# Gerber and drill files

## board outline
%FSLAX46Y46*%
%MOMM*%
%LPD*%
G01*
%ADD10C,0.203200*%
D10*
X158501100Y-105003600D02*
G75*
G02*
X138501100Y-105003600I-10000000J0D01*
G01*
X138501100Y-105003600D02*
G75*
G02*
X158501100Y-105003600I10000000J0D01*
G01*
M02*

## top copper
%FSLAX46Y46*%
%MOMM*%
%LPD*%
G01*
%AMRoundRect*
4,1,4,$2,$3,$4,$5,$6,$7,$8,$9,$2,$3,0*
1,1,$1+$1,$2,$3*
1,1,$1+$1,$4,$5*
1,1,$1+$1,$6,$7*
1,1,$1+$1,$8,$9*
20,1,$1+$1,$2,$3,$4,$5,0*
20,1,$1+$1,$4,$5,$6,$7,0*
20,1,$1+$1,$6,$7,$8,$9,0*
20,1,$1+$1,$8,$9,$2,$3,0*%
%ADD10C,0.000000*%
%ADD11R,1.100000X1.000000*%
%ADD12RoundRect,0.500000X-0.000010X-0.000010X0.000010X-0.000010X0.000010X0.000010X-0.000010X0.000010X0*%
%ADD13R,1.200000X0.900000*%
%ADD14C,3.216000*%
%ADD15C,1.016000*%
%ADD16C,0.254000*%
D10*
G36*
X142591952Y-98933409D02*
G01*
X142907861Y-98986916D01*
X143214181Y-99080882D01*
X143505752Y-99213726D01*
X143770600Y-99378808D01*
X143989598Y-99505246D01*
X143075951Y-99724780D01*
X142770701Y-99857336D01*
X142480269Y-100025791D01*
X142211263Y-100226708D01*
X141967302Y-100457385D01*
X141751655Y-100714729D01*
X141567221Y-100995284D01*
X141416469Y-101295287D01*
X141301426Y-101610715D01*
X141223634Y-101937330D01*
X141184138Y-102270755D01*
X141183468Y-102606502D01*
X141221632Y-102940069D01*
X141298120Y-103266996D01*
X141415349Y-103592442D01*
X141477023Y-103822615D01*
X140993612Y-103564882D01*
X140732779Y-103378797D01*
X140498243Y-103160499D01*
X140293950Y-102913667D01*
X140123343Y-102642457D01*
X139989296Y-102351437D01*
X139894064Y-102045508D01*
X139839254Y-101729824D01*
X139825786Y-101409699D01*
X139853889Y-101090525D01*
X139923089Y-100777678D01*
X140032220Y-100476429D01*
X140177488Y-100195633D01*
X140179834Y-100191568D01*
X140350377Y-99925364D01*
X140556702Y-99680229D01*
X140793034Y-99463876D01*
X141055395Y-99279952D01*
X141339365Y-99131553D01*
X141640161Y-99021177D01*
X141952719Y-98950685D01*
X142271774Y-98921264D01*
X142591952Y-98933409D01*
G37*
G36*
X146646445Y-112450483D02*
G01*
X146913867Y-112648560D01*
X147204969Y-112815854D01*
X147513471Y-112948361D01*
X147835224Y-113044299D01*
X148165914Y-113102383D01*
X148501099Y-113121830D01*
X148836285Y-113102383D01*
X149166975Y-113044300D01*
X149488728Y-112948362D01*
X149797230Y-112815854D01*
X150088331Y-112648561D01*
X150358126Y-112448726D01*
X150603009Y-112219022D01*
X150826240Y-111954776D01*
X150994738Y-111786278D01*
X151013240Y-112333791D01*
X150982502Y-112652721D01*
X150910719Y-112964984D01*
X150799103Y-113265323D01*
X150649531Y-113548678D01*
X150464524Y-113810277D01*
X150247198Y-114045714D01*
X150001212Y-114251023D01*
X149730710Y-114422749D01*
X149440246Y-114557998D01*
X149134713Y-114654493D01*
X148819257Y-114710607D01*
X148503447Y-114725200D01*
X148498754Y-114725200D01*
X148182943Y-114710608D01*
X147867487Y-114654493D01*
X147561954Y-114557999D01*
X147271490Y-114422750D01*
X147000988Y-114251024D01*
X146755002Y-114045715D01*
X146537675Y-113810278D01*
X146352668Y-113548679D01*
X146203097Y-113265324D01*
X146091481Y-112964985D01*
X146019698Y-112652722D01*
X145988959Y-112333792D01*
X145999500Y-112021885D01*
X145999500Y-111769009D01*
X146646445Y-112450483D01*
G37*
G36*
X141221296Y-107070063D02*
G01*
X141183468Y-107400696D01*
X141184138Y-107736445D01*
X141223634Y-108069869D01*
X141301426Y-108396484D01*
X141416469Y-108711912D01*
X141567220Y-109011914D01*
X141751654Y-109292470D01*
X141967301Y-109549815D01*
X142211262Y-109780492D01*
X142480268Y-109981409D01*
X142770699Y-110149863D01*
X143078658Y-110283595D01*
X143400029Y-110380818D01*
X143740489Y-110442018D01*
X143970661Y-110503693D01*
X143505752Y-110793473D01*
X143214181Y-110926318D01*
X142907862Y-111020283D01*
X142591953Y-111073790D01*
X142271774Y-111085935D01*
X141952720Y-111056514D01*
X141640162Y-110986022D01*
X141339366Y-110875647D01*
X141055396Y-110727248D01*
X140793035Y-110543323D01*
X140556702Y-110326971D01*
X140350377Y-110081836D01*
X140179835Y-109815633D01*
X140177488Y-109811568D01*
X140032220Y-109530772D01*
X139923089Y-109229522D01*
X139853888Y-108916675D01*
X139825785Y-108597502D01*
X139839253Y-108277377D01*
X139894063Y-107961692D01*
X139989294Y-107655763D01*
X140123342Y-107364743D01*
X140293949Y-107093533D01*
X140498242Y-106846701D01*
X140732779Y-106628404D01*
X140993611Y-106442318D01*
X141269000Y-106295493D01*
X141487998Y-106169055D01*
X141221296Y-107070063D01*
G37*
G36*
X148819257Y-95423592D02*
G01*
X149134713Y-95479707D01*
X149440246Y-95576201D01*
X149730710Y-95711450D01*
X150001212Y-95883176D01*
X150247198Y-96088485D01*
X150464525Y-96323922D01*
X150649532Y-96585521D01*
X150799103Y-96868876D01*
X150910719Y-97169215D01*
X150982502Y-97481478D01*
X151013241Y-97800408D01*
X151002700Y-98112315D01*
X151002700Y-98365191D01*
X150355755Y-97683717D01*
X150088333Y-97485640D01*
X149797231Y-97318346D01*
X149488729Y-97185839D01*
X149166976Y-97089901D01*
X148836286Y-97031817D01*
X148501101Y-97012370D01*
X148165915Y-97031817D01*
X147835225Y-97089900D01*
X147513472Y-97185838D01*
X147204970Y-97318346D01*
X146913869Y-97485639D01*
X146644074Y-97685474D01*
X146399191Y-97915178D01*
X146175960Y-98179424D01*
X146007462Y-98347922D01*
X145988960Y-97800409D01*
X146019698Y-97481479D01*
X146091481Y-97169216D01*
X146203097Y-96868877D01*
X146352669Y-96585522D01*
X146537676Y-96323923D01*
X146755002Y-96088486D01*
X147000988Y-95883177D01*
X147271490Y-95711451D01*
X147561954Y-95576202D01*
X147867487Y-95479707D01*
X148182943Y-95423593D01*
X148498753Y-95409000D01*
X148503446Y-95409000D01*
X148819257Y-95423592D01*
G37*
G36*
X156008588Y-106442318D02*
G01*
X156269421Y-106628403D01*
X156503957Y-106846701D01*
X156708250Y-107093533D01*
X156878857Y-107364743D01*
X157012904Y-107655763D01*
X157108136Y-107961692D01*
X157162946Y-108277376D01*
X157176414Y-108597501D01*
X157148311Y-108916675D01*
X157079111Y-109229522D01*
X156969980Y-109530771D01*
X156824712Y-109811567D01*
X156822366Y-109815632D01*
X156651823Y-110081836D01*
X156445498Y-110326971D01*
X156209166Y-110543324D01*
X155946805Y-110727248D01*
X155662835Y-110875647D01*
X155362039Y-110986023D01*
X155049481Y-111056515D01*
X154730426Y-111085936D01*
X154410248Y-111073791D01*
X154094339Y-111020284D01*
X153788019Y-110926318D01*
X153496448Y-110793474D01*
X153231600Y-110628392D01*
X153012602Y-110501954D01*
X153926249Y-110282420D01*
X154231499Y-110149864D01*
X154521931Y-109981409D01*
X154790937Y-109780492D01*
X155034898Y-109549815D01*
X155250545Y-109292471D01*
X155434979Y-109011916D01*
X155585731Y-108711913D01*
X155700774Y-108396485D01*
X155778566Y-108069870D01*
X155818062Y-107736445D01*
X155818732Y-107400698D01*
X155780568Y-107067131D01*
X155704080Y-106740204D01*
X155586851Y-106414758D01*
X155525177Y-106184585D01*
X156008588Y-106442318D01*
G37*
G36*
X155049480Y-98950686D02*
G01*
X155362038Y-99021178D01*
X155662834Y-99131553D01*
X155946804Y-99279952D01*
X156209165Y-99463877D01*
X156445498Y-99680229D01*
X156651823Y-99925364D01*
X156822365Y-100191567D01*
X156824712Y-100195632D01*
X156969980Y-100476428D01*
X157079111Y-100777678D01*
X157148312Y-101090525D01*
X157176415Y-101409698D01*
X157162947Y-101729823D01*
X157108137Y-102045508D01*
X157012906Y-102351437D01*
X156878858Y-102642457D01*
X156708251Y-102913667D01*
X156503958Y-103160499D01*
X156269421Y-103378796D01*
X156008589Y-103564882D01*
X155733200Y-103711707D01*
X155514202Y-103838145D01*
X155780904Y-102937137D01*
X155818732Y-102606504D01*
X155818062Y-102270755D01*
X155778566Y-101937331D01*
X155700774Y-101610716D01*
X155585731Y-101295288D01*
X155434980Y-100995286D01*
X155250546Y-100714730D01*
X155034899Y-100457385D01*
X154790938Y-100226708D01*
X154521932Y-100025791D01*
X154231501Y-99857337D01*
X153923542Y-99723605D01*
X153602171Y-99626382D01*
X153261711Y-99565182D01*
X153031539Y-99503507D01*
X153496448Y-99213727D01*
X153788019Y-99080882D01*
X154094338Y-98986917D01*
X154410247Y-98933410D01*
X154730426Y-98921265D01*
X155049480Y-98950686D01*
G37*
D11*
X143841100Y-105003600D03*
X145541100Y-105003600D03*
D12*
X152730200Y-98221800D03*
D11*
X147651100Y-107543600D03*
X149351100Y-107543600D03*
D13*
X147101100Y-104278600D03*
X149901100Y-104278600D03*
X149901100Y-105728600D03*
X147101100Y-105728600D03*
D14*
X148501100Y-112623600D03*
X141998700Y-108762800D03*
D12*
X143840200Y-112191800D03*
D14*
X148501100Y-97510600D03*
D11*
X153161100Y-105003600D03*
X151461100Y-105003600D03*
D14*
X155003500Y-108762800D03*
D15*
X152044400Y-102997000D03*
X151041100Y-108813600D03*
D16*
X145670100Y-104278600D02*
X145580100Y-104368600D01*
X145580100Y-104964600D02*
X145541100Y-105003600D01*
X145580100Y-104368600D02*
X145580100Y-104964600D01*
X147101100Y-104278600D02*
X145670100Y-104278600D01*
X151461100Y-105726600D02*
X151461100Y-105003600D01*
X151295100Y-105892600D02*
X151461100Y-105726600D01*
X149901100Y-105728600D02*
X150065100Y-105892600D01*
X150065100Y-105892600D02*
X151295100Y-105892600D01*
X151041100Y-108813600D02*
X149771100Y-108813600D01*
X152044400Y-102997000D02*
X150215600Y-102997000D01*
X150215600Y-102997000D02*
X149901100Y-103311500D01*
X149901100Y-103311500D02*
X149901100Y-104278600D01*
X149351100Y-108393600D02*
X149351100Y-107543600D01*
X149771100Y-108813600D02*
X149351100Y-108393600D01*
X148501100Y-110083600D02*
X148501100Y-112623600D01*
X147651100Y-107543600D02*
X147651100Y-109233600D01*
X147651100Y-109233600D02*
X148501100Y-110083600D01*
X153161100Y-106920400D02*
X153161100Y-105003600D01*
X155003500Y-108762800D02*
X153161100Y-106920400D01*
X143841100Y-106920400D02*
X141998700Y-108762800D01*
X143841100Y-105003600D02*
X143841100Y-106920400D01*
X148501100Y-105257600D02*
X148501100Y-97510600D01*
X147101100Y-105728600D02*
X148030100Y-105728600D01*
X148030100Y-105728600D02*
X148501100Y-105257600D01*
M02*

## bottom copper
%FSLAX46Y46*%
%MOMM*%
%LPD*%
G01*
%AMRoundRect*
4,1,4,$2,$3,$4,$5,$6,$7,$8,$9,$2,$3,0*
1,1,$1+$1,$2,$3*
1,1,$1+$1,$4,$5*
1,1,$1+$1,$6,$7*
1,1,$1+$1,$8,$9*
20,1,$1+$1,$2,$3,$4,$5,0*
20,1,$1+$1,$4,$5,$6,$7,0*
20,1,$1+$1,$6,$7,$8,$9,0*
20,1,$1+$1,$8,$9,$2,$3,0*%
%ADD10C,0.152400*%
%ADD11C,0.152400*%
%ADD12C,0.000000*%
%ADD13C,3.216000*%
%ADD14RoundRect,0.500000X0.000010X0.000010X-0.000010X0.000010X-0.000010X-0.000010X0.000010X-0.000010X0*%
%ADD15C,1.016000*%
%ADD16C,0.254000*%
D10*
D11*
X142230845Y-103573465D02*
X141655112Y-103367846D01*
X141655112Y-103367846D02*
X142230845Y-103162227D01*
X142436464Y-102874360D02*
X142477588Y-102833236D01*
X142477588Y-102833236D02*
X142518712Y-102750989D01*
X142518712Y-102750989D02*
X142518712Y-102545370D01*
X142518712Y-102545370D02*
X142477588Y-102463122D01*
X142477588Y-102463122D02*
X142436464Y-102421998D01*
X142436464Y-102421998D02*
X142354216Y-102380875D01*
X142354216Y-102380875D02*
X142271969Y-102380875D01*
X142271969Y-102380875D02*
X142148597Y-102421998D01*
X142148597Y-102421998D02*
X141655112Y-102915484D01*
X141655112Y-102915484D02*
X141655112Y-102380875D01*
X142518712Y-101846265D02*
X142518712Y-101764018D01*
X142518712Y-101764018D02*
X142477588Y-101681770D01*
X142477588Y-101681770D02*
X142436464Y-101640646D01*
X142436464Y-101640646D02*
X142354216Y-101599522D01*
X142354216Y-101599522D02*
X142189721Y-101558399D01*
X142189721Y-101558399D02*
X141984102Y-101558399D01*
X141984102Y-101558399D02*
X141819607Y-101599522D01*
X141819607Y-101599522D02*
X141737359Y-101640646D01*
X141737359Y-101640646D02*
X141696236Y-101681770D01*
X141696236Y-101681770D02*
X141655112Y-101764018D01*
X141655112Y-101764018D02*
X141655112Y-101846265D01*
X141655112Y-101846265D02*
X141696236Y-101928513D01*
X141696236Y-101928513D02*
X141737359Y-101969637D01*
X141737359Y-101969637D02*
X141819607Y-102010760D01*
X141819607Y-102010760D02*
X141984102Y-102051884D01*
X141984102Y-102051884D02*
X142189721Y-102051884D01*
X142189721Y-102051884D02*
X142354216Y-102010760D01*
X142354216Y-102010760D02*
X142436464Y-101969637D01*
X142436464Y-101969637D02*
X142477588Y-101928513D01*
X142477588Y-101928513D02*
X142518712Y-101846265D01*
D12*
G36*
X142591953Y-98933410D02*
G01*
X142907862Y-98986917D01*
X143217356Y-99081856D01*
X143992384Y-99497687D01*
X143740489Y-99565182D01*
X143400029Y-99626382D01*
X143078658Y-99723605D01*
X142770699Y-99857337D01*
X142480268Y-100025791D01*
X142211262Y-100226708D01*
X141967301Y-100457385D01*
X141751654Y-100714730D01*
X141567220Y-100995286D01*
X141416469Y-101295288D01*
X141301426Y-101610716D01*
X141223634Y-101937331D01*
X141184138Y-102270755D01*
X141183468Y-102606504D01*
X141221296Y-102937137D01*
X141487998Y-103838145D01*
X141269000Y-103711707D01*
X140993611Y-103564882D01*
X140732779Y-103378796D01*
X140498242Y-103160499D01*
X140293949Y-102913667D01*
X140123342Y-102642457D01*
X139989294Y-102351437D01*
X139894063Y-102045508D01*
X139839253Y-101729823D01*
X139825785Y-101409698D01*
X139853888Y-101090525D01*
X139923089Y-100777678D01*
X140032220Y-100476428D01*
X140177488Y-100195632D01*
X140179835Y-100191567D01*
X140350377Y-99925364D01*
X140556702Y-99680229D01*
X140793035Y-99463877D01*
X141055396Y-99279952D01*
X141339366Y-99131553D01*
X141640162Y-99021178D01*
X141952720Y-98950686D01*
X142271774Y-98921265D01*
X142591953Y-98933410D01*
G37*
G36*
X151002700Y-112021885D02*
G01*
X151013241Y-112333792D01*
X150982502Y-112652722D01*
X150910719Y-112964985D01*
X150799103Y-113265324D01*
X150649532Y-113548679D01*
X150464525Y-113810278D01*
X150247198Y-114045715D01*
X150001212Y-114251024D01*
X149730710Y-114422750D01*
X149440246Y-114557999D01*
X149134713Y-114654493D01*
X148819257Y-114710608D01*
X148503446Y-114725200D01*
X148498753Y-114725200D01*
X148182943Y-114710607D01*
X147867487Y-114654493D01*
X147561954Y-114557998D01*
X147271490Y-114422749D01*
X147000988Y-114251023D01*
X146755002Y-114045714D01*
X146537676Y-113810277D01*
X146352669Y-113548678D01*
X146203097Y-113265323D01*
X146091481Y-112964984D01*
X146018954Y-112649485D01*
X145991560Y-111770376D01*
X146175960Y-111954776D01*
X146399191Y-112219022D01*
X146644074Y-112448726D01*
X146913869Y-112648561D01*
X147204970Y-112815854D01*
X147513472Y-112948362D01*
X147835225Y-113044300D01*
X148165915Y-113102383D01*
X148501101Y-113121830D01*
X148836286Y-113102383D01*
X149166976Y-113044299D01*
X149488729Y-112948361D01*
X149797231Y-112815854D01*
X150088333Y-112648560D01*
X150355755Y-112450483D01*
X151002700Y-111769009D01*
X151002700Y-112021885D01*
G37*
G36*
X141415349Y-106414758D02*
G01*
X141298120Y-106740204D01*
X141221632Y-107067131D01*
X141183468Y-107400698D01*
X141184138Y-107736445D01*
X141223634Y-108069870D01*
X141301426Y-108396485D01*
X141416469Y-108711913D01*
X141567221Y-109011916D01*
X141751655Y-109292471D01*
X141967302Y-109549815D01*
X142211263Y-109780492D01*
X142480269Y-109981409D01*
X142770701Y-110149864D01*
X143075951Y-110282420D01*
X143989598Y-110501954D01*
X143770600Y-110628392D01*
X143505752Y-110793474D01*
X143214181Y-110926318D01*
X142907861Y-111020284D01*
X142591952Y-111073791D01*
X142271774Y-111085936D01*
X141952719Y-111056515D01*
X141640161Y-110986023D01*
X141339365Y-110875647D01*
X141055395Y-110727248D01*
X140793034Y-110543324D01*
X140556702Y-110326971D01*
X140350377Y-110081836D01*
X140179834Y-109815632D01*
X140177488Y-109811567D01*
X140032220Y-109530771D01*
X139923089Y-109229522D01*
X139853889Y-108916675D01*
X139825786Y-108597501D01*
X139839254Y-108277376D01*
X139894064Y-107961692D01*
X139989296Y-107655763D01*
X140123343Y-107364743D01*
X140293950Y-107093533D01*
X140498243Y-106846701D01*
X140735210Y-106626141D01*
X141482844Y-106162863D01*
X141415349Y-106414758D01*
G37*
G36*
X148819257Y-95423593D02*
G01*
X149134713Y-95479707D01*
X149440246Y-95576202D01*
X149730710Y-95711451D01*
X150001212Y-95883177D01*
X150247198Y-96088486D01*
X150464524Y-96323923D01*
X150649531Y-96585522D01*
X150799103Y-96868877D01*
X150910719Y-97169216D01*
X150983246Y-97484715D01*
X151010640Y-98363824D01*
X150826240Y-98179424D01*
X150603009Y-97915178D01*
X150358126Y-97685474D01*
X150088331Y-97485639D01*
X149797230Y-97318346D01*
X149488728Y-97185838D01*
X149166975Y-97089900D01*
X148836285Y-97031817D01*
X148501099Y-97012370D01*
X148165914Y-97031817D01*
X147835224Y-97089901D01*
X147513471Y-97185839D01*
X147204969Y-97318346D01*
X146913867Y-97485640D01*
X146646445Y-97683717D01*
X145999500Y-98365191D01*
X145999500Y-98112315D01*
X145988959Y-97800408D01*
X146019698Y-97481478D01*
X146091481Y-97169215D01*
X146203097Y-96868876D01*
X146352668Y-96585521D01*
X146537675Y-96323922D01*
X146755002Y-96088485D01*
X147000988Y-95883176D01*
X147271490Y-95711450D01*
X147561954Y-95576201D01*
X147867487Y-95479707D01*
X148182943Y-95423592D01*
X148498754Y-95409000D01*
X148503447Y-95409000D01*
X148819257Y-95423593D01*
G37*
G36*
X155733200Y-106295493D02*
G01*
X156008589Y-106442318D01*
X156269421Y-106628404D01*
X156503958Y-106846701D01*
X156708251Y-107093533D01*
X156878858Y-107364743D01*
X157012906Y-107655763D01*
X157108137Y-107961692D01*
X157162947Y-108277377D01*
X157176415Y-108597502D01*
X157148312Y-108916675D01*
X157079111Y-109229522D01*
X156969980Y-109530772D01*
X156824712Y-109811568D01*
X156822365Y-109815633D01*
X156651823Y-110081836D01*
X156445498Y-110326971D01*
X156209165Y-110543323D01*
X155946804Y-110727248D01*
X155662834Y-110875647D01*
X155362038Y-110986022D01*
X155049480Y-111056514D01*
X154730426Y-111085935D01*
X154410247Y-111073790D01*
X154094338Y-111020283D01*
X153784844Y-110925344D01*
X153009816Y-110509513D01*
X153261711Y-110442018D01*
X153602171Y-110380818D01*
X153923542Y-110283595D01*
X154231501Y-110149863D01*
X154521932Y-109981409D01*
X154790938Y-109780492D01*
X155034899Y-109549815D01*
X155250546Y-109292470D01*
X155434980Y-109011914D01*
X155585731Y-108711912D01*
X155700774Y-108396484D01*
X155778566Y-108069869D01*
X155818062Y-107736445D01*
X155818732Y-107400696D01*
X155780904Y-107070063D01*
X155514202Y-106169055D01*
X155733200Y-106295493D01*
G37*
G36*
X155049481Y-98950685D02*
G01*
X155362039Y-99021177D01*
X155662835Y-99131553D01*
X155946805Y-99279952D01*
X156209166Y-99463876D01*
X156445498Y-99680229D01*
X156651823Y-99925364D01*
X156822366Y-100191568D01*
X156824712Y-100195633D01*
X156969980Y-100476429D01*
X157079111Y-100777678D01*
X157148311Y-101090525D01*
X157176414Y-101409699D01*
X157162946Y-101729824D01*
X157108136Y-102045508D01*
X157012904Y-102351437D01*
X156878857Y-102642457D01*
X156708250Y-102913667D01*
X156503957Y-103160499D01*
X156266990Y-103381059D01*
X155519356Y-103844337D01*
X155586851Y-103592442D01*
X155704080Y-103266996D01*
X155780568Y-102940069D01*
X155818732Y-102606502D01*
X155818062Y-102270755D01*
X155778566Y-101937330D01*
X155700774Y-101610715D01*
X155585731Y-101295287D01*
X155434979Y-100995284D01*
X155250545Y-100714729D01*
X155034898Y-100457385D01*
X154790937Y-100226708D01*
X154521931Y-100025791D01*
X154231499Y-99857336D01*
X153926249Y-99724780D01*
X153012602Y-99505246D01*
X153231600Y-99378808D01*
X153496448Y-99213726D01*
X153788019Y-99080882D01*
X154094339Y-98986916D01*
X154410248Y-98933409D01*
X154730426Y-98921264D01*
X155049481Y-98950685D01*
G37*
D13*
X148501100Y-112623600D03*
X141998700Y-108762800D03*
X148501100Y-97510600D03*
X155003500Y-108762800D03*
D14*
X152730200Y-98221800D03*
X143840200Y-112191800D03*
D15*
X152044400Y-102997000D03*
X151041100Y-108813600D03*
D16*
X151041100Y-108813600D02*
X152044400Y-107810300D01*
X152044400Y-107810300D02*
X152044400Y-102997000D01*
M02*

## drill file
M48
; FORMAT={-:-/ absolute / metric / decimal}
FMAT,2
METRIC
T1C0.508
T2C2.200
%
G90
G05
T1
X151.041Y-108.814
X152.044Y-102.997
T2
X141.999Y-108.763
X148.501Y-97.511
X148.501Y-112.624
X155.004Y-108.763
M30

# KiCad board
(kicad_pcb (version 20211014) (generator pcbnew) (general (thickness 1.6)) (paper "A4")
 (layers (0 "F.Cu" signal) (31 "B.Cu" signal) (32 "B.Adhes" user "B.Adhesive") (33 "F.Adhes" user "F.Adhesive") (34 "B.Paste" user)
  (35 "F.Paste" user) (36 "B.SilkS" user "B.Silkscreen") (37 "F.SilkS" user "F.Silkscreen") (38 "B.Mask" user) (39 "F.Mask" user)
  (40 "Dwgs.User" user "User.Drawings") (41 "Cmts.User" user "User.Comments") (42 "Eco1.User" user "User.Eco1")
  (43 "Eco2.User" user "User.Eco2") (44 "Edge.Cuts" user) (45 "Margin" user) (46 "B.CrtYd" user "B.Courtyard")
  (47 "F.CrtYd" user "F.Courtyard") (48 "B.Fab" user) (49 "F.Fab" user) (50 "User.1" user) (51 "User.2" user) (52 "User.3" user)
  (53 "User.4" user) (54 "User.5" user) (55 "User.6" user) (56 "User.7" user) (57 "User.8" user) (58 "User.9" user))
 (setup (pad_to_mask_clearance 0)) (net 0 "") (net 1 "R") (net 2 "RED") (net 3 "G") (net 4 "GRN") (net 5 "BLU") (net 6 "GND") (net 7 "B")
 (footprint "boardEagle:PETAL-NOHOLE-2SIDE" (layer "F.Cu") (at 141.9987 101.2444 -120)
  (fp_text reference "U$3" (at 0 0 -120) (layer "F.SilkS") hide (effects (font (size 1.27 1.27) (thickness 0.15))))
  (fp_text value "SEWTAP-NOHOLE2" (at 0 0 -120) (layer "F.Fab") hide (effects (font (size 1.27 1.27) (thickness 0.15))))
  (fp_poly
   (pts (xy -1.854655 -0.173117) (xy -1.587233 0.02496) (xy -1.296131 0.192254) (xy -0.987629 0.324761) (xy -0.665876 0.420699)
    (xy -0.335186 0.478783) (xy -0.000001 0.49823) (xy 0.335185 0.478783) (xy 0.665875 0.4207) (xy 0.987628 0.324762) (xy 1.29613 0.192254)
    (xy 1.587231 0.024961) (xy 1.857026 -0.174874) (xy 2.101909 -0.404578) (xy 2.32514 -0.668824) (xy 2.493638 -0.837322)
    (xy 2.51214 -0.289809) (xy 2.481402 0.029121) (xy 2.409619 0.341384) (xy 2.298003 0.641723) (xy 2.148431 0.925078)
    (xy 1.963424 1.186677) (xy 1.746098 1.422114) (xy 1.500112 1.627423) (xy 1.22961 1.799149) (xy 0.939146 1.934398) (xy 0.633613 2.030893)
    (xy 0.318157 2.087007) (xy 0.002347 2.1016) (xy -0.002346 2.1016) (xy -0.318157 2.087008) (xy -0.633613 2.030893)
    (xy -0.939146 1.934399) (xy -1.22961 1.79915) (xy -1.500112 1.627424) (xy -1.746098 1.422115) (xy -1.963425 1.186678)
    (xy -2.148432 0.925079) (xy -2.298003 0.641724) (xy -2.409619 0.341385) (xy -2.481402 0.029122) (xy -2.512141 -0.289808)
    (xy -2.5016 -0.601715) (xy -2.5016 -0.854591))
   (layer "F.Cu") (width 0) (fill solid))
  (fp_poly
   (pts (xy 2.5016 -0.601715) (xy 2.512141 -0.289808) (xy 2.481402 0.029122) (xy 2.409619 0.341385) (xy 2.298003 0.641724)
    (xy 2.148432 0.925079) (xy 1.963425 1.186678) (xy 1.746098 1.422115) (xy 1.500112 1.627424) (xy 1.22961 1.79915) (xy 0.939146 1.934399)
    (xy 0.633613 2.030893) (xy 0.318157 2.087008) (xy 0.002346 2.1016) (xy -0.002347 2.1016) (xy -0.318157 2.087007) (xy -0.633613 2.030893)
    (xy -0.939146 1.934398) (xy -1.22961 1.799149) (xy -1.500112 1.627423) (xy -1.746098 1.422114) (xy -1.963424 1.186677)
    (xy -2.148431 0.925078) (xy -2.298003 0.641723) (xy -2.409619 0.341384) (xy -2.482146 0.025885) (xy -2.50954 -0.853224)
    (xy -2.32514 -0.668824) (xy -2.101909 -0.404578) (xy -1.857026 -0.174874) (xy -1.587231 0.024961) (xy -1.29613 0.192254)
    (xy -0.987628 0.324762) (xy -0.665875 0.4207) (xy -0.335185 0.478783) (xy 0.000001 0.49823) (xy 0.335186 0.478783)
    (xy 0.665876 0.420699) (xy 0.987629 0.324761) (xy 1.296131 0.192254) (xy 1.587233 0.02496) (xy 1.854655 -0.173117) (xy 2.5016 -0.854591))
   (layer "B.Cu") (width 0) (fill solid)))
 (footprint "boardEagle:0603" (layer "F.Cu") (at 144.6911 105.0036)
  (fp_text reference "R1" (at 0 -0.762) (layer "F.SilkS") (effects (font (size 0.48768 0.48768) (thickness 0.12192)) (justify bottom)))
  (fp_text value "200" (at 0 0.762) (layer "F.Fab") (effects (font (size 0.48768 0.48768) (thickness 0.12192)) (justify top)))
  (pad "1" smd rect (at -0.85 0) (size 1.1 1) (layers "F.Cu" "F.Paste" "F.Mask") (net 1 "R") (solder_mask_margin 0.1016))
  (pad "2" smd rect (at 0.85 0) (size 1.1 1) (layers "F.Cu" "F.Paste" "F.Mask") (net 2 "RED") (solder_mask_margin 0.1016)))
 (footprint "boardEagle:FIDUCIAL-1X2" (layer "F.Cu") (at 152.7302 98.2218)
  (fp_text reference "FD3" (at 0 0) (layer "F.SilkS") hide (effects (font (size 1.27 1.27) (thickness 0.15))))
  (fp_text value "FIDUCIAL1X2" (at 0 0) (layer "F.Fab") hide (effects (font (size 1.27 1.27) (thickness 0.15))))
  (pad "1" smd roundrect (at 0 0) (size 1 1) (layers "F.Cu" "F.Mask") (roundrect_rratio 0.5) (solder_mask_margin 0.1016)))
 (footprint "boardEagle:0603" (layer "F.Cu") (at 148.5011 107.5436)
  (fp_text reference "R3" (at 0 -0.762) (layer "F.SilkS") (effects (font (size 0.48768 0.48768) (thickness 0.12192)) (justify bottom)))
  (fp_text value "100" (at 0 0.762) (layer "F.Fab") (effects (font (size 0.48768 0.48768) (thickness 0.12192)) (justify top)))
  (pad "1" smd rect (at -0.85 0) (size 1.1 1) (layers "F.Cu" "F.Paste" "F.Mask") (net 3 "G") (solder_mask_margin 0.1016))
  (pad "2" smd rect (at 0.85 0) (size 1.1 1) (layers "F.Cu" "F.Paste" "F.Mask") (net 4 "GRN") (solder_mask_margin 0.1016)))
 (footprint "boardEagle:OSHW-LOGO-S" (layer "F.Cu") (at 143.9291 102.4636)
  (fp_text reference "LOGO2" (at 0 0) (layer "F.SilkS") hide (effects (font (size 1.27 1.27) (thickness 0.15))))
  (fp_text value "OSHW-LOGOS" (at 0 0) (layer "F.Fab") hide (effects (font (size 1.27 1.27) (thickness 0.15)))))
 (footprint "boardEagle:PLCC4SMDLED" (layer "F.Cu") (at 148.5011 105.0036)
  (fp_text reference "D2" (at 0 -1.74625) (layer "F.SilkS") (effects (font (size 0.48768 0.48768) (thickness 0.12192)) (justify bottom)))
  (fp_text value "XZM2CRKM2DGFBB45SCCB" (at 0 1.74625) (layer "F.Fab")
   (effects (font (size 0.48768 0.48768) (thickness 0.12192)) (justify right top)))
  (pad "1" smd rect (at -1.4 -0.725) (size 1.2 0.9) (layers "F.Cu" "F.Paste" "F.Mask") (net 2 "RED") (solder_mask_margin 0.1016))
  (pad "2" smd rect (at 1.4 -0.725) (size 1.2 0.9) (layers "F.Cu" "F.Paste" "F.Mask") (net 4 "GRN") (solder_mask_margin 0.1016))
  (pad "3" smd rect (at 1.4 0.725) (size 1.2 0.9) (layers "F.Cu" "F.Paste" "F.Mask") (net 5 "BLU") (solder_mask_margin 0.1016))
  (pad "4" smd rect (at -1.4 0.725) (size 1.2 0.9) (layers "F.Cu" "F.Paste" "F.Mask") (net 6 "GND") (solder_mask_margin 0.1016)))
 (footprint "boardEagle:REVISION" (layer "F.Cu") (at 129.8702 129.9718)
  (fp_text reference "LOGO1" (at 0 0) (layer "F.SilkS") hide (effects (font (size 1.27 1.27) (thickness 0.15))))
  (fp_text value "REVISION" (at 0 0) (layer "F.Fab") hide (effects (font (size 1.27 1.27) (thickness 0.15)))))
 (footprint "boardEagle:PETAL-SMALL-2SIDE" (layer "F.Cu") (at 148.5011 112.6236)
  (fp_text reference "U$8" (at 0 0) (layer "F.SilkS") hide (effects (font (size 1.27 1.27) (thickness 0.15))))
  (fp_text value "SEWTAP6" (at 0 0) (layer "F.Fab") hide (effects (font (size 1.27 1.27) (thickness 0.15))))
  (fp_poly
   (pts (xy -1.854655 -0.173117) (xy -1.587233 0.02496) (xy -1.296131 0.192254) (xy -0.987629 0.324761) (xy -0.665876 0.420699)
    (xy -0.335186 0.478783) (xy -0.000001 0.49823) (xy 0.335185 0.478783) (xy 0.665875 0.4207) (xy 0.987628 0.324762) (xy 1.29613 0.192254)
    (xy 1.587231 0.024961) (xy 1.857026 -0.174874) (xy 2.101909 -0.404578) (xy 2.32514 -0.668824) (xy 2.493638 -0.837322)
    (xy 2.51214 -0.289809) (xy 2.481402 0.029121) (xy 2.409619 0.341384) (xy 2.298003 0.641723) (xy 2.148431 0.925078)
    (xy 1.963424 1.186677) (xy 1.746098 1.422114) (xy 1.500112 1.627423) (xy 1.22961 1.799149) (xy 0.939146 1.934398) (xy 0.633613 2.030893)
    (xy 0.318157 2.087007) (xy 0.002347 2.1016) (xy -0.002346 2.1016) (xy -0.318157 2.087008) (xy -0.633613 2.030893)
    (xy -0.939146 1.934399) (xy -1.22961 1.79915) (xy -1.500112 1.627424) (xy -1.746098 1.422115) (xy -1.963425 1.186678)
    (xy -2.148432 0.925079) (xy -2.298003 0.641724) (xy -2.409619 0.341385) (xy -2.481402 0.029122) (xy -2.512141 -0.289808)
    (xy -2.5016 -0.601715) (xy -2.5016 -0.854591))
   (layer "F.Cu") (width 0) (fill solid))
  (fp_poly
   (pts (xy 2.5016 -0.601715) (xy 2.512141 -0.289808) (xy 2.481402 0.029122) (xy 2.409619 0.341385) (xy 2.298003 0.641724)
    (xy 2.148432 0.925079) (xy 1.963425 1.186678) (xy 1.746098 1.422115) (xy 1.500112 1.627424) (xy 1.22961 1.79915) (xy 0.939146 1.934399)
    (xy 0.633613 2.030893) (xy 0.318157 2.087008) (xy 0.002346 2.1016) (xy -0.002347 2.1016) (xy -0.318157 2.087007) (xy -0.633613 2.030893)
    (xy -0.939146 1.934398) (xy -1.22961 1.799149) (xy -1.500112 1.627423) (xy -1.746098 1.422114) (xy -1.963424 1.186677)
    (xy -2.148431 0.925078) (xy -2.298003 0.641723) (xy -2.409619 0.341384) (xy -2.482146 0.025885) (xy -2.50954 -0.853224)
    (xy -2.32514 -0.668824) (xy -2.101909 -0.404578) (xy -1.857026 -0.174874) (xy -1.587231 0.024961) (xy -1.29613 0.192254)
    (xy -0.987628 0.324762) (xy -0.665875 0.4207) (xy -0.335185 0.478783) (xy 0.000001 0.49823) (xy 0.335186 0.478783)
    (xy 0.665876 0.420699) (xy 0.987629 0.324761) (xy 1.296131 0.192254) (xy 1.587233 0.02496) (xy 1.854655 -0.173117) (xy 2.5016 -0.854591))
   (layer "B.Cu") (width 0) (fill solid))
  (pad "1" thru_hole circle (at 0 0 90) (size 3.216 3.216) (drill 2.2) (layers *.Cu *.Mask) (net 3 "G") (solder_mask_margin 0.1016)))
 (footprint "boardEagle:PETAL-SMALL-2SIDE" (layer "F.Cu") (at 141.9987 108.7628 -60)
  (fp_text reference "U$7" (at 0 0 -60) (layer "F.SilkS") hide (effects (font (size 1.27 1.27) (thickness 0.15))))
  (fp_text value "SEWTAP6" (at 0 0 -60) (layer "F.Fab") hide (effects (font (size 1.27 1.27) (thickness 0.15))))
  (fp_poly
   (pts (xy -1.854655 -0.173117) (xy -1.587233 0.02496) (xy -1.296131 0.192254) (xy -0.987629 0.324761) (xy -0.665876 0.420699)
    (xy -0.335186 0.478783) (xy -0.000001 0.49823) (xy 0.335185 0.478783) (xy 0.665875 0.4207) (xy 0.987628 0.324762) (xy 1.29613 0.192254)
    (xy 1.587231 0.024961) (xy 1.857026 -0.174874) (xy 2.101909 -0.404578) (xy 2.32514 -0.668824) (xy 2.493638 -0.837322)
    (xy 2.51214 -0.289809) (xy 2.481402 0.029121) (xy 2.409619 0.341384) (xy 2.298003 0.641723) (xy 2.148431 0.925078)
    (xy 1.963424 1.186677) (xy 1.746098 1.422114) (xy 1.500112 1.627423) (xy 1.22961 1.799149) (xy 0.939146 1.934398) (xy 0.633613 2.030893)
    (xy 0.318157 2.087007) (xy 0.002347 2.1016) (xy -0.002346 2.1016) (xy -0.318157 2.087008) (xy -0.633613 2.030893)
    (xy -0.939146 1.934399) (xy -1.22961 1.79915) (xy -1.500112 1.627424) (xy -1.746098 1.422115) (xy -1.963425 1.186678)
    (xy -2.148432 0.925079) (xy -2.298003 0.641724) (xy -2.409619 0.341385) (xy -2.481402 0.029122) (xy -2.512141 -0.289808)
    (xy -2.5016 -0.601715) (xy -2.5016 -0.854591))
   (layer "F.Cu") (width 0) (fill solid))
  (fp_poly
   (pts (xy 2.5016 -0.601715) (xy 2.512141 -0.289808) (xy 2.481402 0.029122) (xy 2.409619 0.341385) (xy 2.298003 0.641724)
    (xy 2.148432 0.925079) (xy 1.963425 1.186678) (xy 1.746098 1.422115) (xy 1.500112 1.627424) (xy 1.22961 1.79915) (xy 0.939146 1.934399)
    (xy 0.633613 2.030893) (xy 0.318157 2.087008) (xy 0.002346 2.1016) (xy -0.002347 2.1016) (xy -0.318157 2.087007) (xy -0.633613 2.030893)
    (xy -0.939146 1.934398) (xy -1.22961 1.799149) (xy -1.500112 1.627423) (xy -1.746098 1.422114) (xy -1.963424 1.186677)
    (xy -2.148431 0.925078) (xy -2.298003 0.641723) (xy -2.409619 0.341384) (xy -2.482146 0.025885) (xy -2.50954 -0.853224)
    (xy -2.32514 -0.668824) (xy -2.101909 -0.404578) (xy -1.857026 -0.174874) (xy -1.587231 0.024961) (xy -1.29613 0.192254)
    (xy -0.987628 0.324762) (xy -0.665875 0.4207) (xy -0.335185 0.478783) (xy 0.000001 0.49823) (xy 0.335186 0.478783)
    (xy 0.665876 0.420699) (xy 0.987629 0.324761) (xy 1.296131 0.192254) (xy 1.587233 0.02496) (xy 1.854655 -0.173117) (xy 2.5016 -0.854591))
   (layer "B.Cu") (width 0) (fill solid))
  (pad "1" thru_hole circle (at 0 0 30) (size 3.216 3.216) (drill 2.2) (layers *.Cu *.Mask) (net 1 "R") (solder_mask_margin 0.1016)))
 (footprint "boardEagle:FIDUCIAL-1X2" (layer "F.Cu") (at 143.8402 112.1918)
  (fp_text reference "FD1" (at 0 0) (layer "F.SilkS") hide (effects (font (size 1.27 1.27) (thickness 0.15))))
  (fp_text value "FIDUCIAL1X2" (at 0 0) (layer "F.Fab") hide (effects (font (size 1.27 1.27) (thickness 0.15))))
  (pad "1" smd roundrect (at 0 0) (size 1 1) (layers "F.Cu" "F.Mask") (roundrect_rratio 0.5) (solder_mask_margin 0.1016)))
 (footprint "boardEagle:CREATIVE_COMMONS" (layer "F.Cu") (at 118.619144 127.4318)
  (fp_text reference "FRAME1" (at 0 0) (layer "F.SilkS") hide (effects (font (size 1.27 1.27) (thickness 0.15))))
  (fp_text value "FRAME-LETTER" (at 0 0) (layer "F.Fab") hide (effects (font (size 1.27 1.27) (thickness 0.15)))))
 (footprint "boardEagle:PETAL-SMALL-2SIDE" (layer "F.Cu") (at 148.5011 97.5106 180)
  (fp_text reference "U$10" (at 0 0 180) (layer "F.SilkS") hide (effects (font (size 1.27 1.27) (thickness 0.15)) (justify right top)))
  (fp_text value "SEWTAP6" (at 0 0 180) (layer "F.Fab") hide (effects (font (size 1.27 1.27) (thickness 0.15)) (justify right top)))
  (fp_poly
   (pts (xy -1.854655 -0.173117) (xy -1.587233 0.02496) (xy -1.296131 0.192254) (xy -0.987629 0.324761) (xy -0.665876 0.420699)
    (xy -0.335186 0.478783) (xy -0.000001 0.49823) (xy 0.335185 0.478783) (xy 0.665875 0.4207) (xy 0.987628 0.324762) (xy 1.29613 0.192254)
    (xy 1.587231 0.024961) (xy 1.857026 -0.174874) (xy 2.101909 -0.404578) (xy 2.32514 -0.668824) (xy 2.493638 -0.837322)
    (xy 2.51214 -0.289809) (xy 2.481402 0.029121) (xy 2.409619 0.341384) (xy 2.298003 0.641723) (xy 2.148431 0.925078)
    (xy 1.963424 1.186677) (xy 1.746098 1.422114) (xy 1.500112 1.627423) (xy 1.22961 1.799149) (xy 0.939146 1.934398) (xy 0.633613 2.030893)
    (xy 0.318157 2.087007) (xy 0.002347 2.1016) (xy -0.002346 2.1016) (xy -0.318157 2.087008) (xy -0.633613 2.030893)
    (xy -0.939146 1.934399) (xy -1.22961 1.79915) (xy -1.500112 1.627424) (xy -1.746098 1.422115) (xy -1.963425 1.186678)
    (xy -2.148432 0.925079) (xy -2.298003 0.641724) (xy -2.409619 0.341385) (xy -2.481402 0.029122) (xy -2.512141 -0.289808)
    (xy -2.5016 -0.601715) (xy -2.5016 -0.854591))
   (layer "F.Cu") (width 0) (fill solid))
  (fp_poly
   (pts (xy 2.5016 -0.601715) (xy 2.512141 -0.289808) (xy 2.481402 0.029122) (xy 2.409619 0.341385) (xy 2.298003 0.641724)
    (xy 2.148432 0.925079) (xy 1.963425 1.186678) (xy 1.746098 1.422115) (xy 1.500112 1.627424) (xy 1.22961 1.79915) (xy 0.939146 1.934399)
    (xy 0.633613 2.030893) (xy 0.318157 2.087008) (xy 0.002346 2.1016) (xy -0.002347 2.1016) (xy -0.318157 2.087007) (xy -0.633613 2.030893)
    (xy -0.939146 1.934398) (xy -1.22961 1.799149) (xy -1.500112 1.627423) (xy -1.746098 1.422114) (xy -1.963424 1.186677)
    (xy -2.148431 0.925078) (xy -2.298003 0.641723) (xy -2.409619 0.341384) (xy -2.482146 0.025885) (xy -2.50954 -0.853224)
    (xy -2.32514 -0.668824) (xy -2.101909 -0.404578) (xy -1.857026 -0.174874) (xy -1.587231 0.024961) (xy -1.29613 0.192254)
    (xy -0.987628 0.324762) (xy -0.665875 0.4207) (xy -0.335185 0.478783) (xy 0.000001 0.49823) (xy 0.335186 0.478783)
    (xy 0.665876 0.420699) (xy 0.987629 0.324761) (xy 1.296131 0.192254) (xy 1.587233 0.02496) (xy 1.854655 -0.173117) (xy 2.5016 -0.854591))
   (layer "B.Cu") (width 0) (fill solid))
  (pad "1" thru_hole circle (at 0 0 270) (size 3.216 3.216) (drill 2.2) (layers *.Cu *.Mask) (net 6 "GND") (solder_mask_margin 0.1016)))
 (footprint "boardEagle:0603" (layer "F.Cu") (at 152.3111 105.0036 180)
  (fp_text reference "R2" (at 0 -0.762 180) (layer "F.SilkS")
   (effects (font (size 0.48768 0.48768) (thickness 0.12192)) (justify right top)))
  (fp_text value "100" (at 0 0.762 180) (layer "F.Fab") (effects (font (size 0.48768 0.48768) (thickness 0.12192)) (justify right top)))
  (pad "1" smd rect (at -0.85 0 180) (size 1.1 1) (layers "F.Cu" "F.Paste" "F.Mask") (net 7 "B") (solder_mask_margin 0.1016))
  (pad "2" smd rect (at 0.85 0 180) (size 1.1 1) (layers "F.Cu" "F.Paste" "F.Mask") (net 5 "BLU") (solder_mask_margin 0.1016)))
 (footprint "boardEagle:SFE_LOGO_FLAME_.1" (layer "F.Cu") (at 152.4381 103.7336)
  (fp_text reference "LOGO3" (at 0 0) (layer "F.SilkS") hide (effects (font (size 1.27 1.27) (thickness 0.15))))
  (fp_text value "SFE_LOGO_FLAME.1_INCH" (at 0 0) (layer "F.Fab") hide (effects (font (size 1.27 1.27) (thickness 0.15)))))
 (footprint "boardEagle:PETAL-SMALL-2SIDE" (layer "F.Cu") (at 155.0035 108.7628 60)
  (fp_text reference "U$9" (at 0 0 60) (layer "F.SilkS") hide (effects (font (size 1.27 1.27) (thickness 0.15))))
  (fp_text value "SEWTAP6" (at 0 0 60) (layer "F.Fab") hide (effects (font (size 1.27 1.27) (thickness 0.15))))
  (fp_poly
   (pts (xy -1.854655 -0.173117) (xy -1.587233 0.02496) (xy -1.296131 0.192254) (xy -0.987629 0.324761) (xy -0.665876 0.420699)
    (xy -0.335186 0.478783) (xy -0.000001 0.49823) (xy 0.335185 0.478783) (xy 0.665875 0.4207) (xy 0.987628 0.324762) (xy 1.29613 0.192254)
    (xy 1.587231 0.024961) (xy 1.857026 -0.174874) (xy 2.101909 -0.404578) (xy 2.32514 -0.668824) (xy 2.493638 -0.837322)
    (xy 2.51214 -0.289809) (xy 2.481402 0.029121) (xy 2.409619 0.341384) (xy 2.298003 0.641723) (xy 2.148431 0.925078)
    (xy 1.963424 1.186677) (xy 1.746098 1.422114) (xy 1.500112 1.627423) (xy 1.22961 1.799149) (xy 0.939146 1.934398) (xy 0.633613 2.030893)
    (xy 0.318157 2.087007) (xy 0.002347 2.1016) (xy -0.002346 2.1016) (xy -0.318157 2.087008) (xy -0.633613 2.030893)
    (xy -0.939146 1.934399) (xy -1.22961 1.79915) (xy -1.500112 1.627424) (xy -1.746098 1.422115) (xy -1.963425 1.186678)
    (xy -2.148432 0.925079) (xy -2.298003 0.641724) (xy -2.409619 0.341385) (xy -2.481402 0.029122) (xy -2.512141 -0.289808)
    (xy -2.5016 -0.601715) (xy -2.5016 -0.854591))
   (layer "F.Cu") (width 0) (fill solid))
  (fp_poly
   (pts (xy 2.5016 -0.601715) (xy 2.512141 -0.289808) (xy 2.481402 0.029122) (xy 2.409619 0.341385) (xy 2.298003 0.641724)
    (xy 2.148432 0.925079) (xy 1.963425 1.186678) (xy 1.746098 1.422115) (xy 1.500112 1.627424) (xy 1.22961 1.79915) (xy 0.939146 1.934399)
    (xy 0.633613 2.030893) (xy 0.318157 2.087008) (xy 0.002346 2.1016) (xy -0.002347 2.1016) (xy -0.318157 2.087007) (xy -0.633613 2.030893)
    (xy -0.939146 1.934398) (xy -1.22961 1.799149) (xy -1.500112 1.627423) (xy -1.746098 1.422114) (xy -1.963424 1.186677)
    (xy -2.148431 0.925078) (xy -2.298003 0.641723) (xy -2.409619 0.341384) (xy -2.482146 0.025885) (xy -2.50954 -0.853224)
    (xy -2.32514 -0.668824) (xy -2.101909 -0.404578) (xy -1.857026 -0.174874) (xy -1.587231 0.024961) (xy -1.29613 0.192254)
    (xy -0.987628 0.324762) (xy -0.665875 0.4207) (xy -0.335185 0.478783) (xy 0.000001 0.49823) (xy 0.335186 0.478783)
    (xy 0.665876 0.420699) (xy 0.987629 0.324761) (xy 1.296131 0.192254) (xy 1.587233 0.02496) (xy 1.854655 -0.173117) (xy 2.5016 -0.854591))
   (layer "B.Cu") (width 0) (fill solid))
  (pad "1" thru_hole circle (at 0 0 150) (size 3.216 3.216) (drill 2.2) (layers *.Cu *.Mask) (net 7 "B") (solder_mask_margin 0.1016)))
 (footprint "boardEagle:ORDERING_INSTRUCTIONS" (layer "F.Cu") (at 127.3302 131.2418)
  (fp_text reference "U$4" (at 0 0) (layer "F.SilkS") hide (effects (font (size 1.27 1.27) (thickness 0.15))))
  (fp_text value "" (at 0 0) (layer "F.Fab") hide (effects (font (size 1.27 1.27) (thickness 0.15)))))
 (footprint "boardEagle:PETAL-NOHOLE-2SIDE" (layer "F.Cu") (at 155.0035 101.2444 120)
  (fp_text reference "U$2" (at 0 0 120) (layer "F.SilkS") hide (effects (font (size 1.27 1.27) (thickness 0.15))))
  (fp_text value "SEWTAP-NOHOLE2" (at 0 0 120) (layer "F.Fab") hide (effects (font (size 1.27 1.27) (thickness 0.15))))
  (fp_poly
   (pts (xy -1.854655 -0.173117) (xy -1.587233 0.02496) (xy -1.296131 0.192254) (xy -0.987629 0.324761) (xy -0.665876 0.420699)
    (xy -0.335186 0.478783) (xy -0.000001 0.49823) (xy 0.335185 0.478783) (xy 0.665875 0.4207) (xy 0.987628 0.324762) (xy 1.29613 0.192254)
    (xy 1.587231 0.024961) (xy 1.857026 -0.174874) (xy 2.101909 -0.404578) (xy 2.32514 -0.668824) (xy 2.493638 -0.837322)
    (xy 2.51214 -0.289809) (xy 2.481402 0.029121) (xy 2.409619 0.341384) (xy 2.298003 0.641723) (xy 2.148431 0.925078)
    (xy 1.963424 1.186677) (xy 1.746098 1.422114) (xy 1.500112 1.627423) (xy 1.22961 1.799149) (xy 0.939146 1.934398) (xy 0.633613 2.030893)
    (xy 0.318157 2.087007) (xy 0.002347 2.1016) (xy -0.002346 2.1016) (xy -0.318157 2.087008) (xy -0.633613 2.030893)
    (xy -0.939146 1.934399) (xy -1.22961 1.79915) (xy -1.500112 1.627424) (xy -1.746098 1.422115) (xy -1.963425 1.186678)
    (xy -2.148432 0.925079) (xy -2.298003 0.641724) (xy -2.409619 0.341385) (xy -2.481402 0.029122) (xy -2.512141 -0.289808)
    (xy -2.5016 -0.601715) (xy -2.5016 -0.854591))
   (layer "F.Cu") (width 0) (fill solid))
  (fp_poly
   (pts (xy 2.5016 -0.601715) (xy 2.512141 -0.289808) (xy 2.481402 0.029122) (xy 2.409619 0.341385) (xy 2.298003 0.641724)
    (xy 2.148432 0.925079) (xy 1.963425 1.186678) (xy 1.746098 1.422115) (xy 1.500112 1.627424) (xy 1.22961 1.79915) (xy 0.939146 1.934399)
    (xy 0.633613 2.030893) (xy 0.318157 2.087008) (xy 0.002346 2.1016) (xy -0.002347 2.1016) (xy -0.318157 2.087007) (xy -0.633613 2.030893)
    (xy -0.939146 1.934398) (xy -1.22961 1.799149) (xy -1.500112 1.627423) (xy -1.746098 1.422114) (xy -1.963424 1.186677)
    (xy -2.148431 0.925078) (xy -2.298003 0.641723) (xy -2.409619 0.341384) (xy -2.482146 0.025885) (xy -2.50954 -0.853224)
    (xy -2.32514 -0.668824) (xy -2.101909 -0.404578) (xy -1.857026 -0.174874) (xy -1.587231 0.024961) (xy -1.29613 0.192254)
    (xy -0.987628 0.324762) (xy -0.665875 0.4207) (xy -0.335185 0.478783) (xy 0.000001 0.49823) (xy 0.335186 0.478783)
    (xy 0.665876 0.420699) (xy 0.987629 0.324761) (xy 1.296131 0.192254) (xy 1.587233 0.02496) (xy 1.854655 -0.173117) (xy 2.5016 -0.854591))
   (layer "B.Cu") (width 0) (fill solid)))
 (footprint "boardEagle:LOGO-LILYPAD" (layer "B.Cu") (at 148.5011 104.7496 180)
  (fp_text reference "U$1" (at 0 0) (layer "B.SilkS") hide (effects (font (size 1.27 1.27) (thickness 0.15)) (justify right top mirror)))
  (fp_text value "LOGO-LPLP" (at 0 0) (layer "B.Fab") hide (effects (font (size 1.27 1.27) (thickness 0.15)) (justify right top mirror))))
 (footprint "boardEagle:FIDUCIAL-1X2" (layer "B.Cu") (at 152.7302 98.2218 180)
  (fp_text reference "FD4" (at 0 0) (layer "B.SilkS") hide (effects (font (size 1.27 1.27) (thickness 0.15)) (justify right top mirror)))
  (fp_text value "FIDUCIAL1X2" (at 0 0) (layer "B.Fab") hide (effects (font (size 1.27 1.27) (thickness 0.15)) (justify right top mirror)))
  (pad "1" smd roundrect (at 0 0 180) (size 1 1) (layers "B.Cu" "B.Mask") (roundrect_rratio 0.5) (solder_mask_margin 0.1016)))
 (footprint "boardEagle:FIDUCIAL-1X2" (layer "B.Cu") (at 143.8402 112.1918 180)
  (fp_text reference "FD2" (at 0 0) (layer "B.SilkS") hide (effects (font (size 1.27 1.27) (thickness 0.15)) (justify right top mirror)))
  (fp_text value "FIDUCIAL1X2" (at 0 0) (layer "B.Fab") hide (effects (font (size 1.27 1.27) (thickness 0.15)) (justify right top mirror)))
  (pad "1" smd roundrect (at 0 0 180) (size 1 1) (layers "B.Cu" "B.Mask") (roundrect_rratio 0.5) (solder_mask_margin 0.1016)))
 (gr_circle (center 148.5011 105.0036) (end 158.5011 105.0036) (layer "Edge.Cuts") (width 0.2032) (fill none))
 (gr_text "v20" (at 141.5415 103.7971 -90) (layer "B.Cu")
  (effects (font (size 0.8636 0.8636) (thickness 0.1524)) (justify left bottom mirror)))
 (segment (start 145.6701 104.2786) (end 145.5801 104.3686) (width 0.254) (layer "F.Cu") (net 2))
 (segment (start 145.5801 104.9646) (end 145.5411 105.0036) (width 0.254) (layer "F.Cu") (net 2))
 (segment (start 145.5801 104.3686) (end 145.5801 104.9646) (width 0.254) (layer "F.Cu") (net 2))
 (segment (start 147.1011 104.2786) (end 145.6701 104.2786) (width 0.254) (layer "F.Cu") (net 2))
 (segment (start 151.4611 105.7266) (end 151.4611 105.0036) (width 0.254) (layer "F.Cu") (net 5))
 (segment (start 151.2951 105.8926) (end 151.4611 105.7266) (width 0.254) (layer "F.Cu") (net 5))
 (segment (start 149.9011 105.7286) (end 150.0651 105.8926) (width 0.254) (layer "F.Cu") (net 5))
 (segment (start 150.0651 105.8926) (end 151.2951 105.8926) (width 0.254) (layer "F.Cu") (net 5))
 (segment (start 151.0411 108.8136) (end 149.7711 108.8136) (width 0.254) (layer "F.Cu") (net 4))
 (segment (start 152.0444 102.997) (end 150.2156 102.997) (width 0.254) (layer "F.Cu") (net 4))
 (segment (start 150.2156 102.997) (end 149.9011 103.3115) (width 0.254) (layer "F.Cu") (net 4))
 (segment (start 149.9011 103.3115) (end 149.9011 104.2786) (width 0.254) (layer "F.Cu") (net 4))
 (segment (start 149.3511 108.3936) (end 149.3511 107.5436) (width 0.254) (layer "F.Cu") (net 4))
 (segment (start 149.7711 108.8136) (end 149.3511 108.3936) (width 0.254) (layer "F.Cu") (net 4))
 (via (at 152.0444 102.997) (size 1.016) (drill 0.508) (layers "F.Cu" "B.Cu") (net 4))
 (via (at 151.0411 108.8136) (size 1.016) (drill 0.508) (layers "F.Cu" "B.Cu") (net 4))
 (segment (start 151.0411 108.8136) (end 152.0444 107.8103) (width 0.254) (layer "B.Cu") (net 4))
 (segment (start 152.0444 107.8103) (end 152.0444 102.997) (width 0.254) (layer "B.Cu") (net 4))
 (segment (start 148.5011 110.0836) (end 148.5011 112.6236) (width 0.254) (layer "F.Cu") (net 3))
 (segment (start 147.6511 107.5436) (end 147.6511 109.2336) (width 0.254) (layer "F.Cu") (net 3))
 (segment (start 147.6511 109.2336) (end 148.5011 110.0836) (width 0.254) (layer "F.Cu") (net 3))
 (segment (start 153.1611 106.9204) (end 153.1611 105.0036) (width 0.254) (layer "F.Cu") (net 7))
 (segment (start 155.0035 108.7628) (end 153.1611 106.9204) (width 0.254) (layer "F.Cu") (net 7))
 (segment (start 143.8411 106.9204) (end 141.9987 108.7628) (width 0.254) (layer "F.Cu") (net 1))
 (segment (start 143.8411 105.0036) (end 143.8411 106.9204) (width 0.254) (layer "F.Cu") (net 1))
 (segment (start 148.5011 105.2576) (end 148.5011 97.5106) (width 0.254) (layer "F.Cu") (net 6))
 (segment (start 147.1011 105.7286) (end 148.0301 105.7286) (width 0.254) (layer "F.Cu") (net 6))
 (segment (start 148.0301 105.7286) (end 148.5011 105.2576) (width 0.254) (layer "F.Cu") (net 6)))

